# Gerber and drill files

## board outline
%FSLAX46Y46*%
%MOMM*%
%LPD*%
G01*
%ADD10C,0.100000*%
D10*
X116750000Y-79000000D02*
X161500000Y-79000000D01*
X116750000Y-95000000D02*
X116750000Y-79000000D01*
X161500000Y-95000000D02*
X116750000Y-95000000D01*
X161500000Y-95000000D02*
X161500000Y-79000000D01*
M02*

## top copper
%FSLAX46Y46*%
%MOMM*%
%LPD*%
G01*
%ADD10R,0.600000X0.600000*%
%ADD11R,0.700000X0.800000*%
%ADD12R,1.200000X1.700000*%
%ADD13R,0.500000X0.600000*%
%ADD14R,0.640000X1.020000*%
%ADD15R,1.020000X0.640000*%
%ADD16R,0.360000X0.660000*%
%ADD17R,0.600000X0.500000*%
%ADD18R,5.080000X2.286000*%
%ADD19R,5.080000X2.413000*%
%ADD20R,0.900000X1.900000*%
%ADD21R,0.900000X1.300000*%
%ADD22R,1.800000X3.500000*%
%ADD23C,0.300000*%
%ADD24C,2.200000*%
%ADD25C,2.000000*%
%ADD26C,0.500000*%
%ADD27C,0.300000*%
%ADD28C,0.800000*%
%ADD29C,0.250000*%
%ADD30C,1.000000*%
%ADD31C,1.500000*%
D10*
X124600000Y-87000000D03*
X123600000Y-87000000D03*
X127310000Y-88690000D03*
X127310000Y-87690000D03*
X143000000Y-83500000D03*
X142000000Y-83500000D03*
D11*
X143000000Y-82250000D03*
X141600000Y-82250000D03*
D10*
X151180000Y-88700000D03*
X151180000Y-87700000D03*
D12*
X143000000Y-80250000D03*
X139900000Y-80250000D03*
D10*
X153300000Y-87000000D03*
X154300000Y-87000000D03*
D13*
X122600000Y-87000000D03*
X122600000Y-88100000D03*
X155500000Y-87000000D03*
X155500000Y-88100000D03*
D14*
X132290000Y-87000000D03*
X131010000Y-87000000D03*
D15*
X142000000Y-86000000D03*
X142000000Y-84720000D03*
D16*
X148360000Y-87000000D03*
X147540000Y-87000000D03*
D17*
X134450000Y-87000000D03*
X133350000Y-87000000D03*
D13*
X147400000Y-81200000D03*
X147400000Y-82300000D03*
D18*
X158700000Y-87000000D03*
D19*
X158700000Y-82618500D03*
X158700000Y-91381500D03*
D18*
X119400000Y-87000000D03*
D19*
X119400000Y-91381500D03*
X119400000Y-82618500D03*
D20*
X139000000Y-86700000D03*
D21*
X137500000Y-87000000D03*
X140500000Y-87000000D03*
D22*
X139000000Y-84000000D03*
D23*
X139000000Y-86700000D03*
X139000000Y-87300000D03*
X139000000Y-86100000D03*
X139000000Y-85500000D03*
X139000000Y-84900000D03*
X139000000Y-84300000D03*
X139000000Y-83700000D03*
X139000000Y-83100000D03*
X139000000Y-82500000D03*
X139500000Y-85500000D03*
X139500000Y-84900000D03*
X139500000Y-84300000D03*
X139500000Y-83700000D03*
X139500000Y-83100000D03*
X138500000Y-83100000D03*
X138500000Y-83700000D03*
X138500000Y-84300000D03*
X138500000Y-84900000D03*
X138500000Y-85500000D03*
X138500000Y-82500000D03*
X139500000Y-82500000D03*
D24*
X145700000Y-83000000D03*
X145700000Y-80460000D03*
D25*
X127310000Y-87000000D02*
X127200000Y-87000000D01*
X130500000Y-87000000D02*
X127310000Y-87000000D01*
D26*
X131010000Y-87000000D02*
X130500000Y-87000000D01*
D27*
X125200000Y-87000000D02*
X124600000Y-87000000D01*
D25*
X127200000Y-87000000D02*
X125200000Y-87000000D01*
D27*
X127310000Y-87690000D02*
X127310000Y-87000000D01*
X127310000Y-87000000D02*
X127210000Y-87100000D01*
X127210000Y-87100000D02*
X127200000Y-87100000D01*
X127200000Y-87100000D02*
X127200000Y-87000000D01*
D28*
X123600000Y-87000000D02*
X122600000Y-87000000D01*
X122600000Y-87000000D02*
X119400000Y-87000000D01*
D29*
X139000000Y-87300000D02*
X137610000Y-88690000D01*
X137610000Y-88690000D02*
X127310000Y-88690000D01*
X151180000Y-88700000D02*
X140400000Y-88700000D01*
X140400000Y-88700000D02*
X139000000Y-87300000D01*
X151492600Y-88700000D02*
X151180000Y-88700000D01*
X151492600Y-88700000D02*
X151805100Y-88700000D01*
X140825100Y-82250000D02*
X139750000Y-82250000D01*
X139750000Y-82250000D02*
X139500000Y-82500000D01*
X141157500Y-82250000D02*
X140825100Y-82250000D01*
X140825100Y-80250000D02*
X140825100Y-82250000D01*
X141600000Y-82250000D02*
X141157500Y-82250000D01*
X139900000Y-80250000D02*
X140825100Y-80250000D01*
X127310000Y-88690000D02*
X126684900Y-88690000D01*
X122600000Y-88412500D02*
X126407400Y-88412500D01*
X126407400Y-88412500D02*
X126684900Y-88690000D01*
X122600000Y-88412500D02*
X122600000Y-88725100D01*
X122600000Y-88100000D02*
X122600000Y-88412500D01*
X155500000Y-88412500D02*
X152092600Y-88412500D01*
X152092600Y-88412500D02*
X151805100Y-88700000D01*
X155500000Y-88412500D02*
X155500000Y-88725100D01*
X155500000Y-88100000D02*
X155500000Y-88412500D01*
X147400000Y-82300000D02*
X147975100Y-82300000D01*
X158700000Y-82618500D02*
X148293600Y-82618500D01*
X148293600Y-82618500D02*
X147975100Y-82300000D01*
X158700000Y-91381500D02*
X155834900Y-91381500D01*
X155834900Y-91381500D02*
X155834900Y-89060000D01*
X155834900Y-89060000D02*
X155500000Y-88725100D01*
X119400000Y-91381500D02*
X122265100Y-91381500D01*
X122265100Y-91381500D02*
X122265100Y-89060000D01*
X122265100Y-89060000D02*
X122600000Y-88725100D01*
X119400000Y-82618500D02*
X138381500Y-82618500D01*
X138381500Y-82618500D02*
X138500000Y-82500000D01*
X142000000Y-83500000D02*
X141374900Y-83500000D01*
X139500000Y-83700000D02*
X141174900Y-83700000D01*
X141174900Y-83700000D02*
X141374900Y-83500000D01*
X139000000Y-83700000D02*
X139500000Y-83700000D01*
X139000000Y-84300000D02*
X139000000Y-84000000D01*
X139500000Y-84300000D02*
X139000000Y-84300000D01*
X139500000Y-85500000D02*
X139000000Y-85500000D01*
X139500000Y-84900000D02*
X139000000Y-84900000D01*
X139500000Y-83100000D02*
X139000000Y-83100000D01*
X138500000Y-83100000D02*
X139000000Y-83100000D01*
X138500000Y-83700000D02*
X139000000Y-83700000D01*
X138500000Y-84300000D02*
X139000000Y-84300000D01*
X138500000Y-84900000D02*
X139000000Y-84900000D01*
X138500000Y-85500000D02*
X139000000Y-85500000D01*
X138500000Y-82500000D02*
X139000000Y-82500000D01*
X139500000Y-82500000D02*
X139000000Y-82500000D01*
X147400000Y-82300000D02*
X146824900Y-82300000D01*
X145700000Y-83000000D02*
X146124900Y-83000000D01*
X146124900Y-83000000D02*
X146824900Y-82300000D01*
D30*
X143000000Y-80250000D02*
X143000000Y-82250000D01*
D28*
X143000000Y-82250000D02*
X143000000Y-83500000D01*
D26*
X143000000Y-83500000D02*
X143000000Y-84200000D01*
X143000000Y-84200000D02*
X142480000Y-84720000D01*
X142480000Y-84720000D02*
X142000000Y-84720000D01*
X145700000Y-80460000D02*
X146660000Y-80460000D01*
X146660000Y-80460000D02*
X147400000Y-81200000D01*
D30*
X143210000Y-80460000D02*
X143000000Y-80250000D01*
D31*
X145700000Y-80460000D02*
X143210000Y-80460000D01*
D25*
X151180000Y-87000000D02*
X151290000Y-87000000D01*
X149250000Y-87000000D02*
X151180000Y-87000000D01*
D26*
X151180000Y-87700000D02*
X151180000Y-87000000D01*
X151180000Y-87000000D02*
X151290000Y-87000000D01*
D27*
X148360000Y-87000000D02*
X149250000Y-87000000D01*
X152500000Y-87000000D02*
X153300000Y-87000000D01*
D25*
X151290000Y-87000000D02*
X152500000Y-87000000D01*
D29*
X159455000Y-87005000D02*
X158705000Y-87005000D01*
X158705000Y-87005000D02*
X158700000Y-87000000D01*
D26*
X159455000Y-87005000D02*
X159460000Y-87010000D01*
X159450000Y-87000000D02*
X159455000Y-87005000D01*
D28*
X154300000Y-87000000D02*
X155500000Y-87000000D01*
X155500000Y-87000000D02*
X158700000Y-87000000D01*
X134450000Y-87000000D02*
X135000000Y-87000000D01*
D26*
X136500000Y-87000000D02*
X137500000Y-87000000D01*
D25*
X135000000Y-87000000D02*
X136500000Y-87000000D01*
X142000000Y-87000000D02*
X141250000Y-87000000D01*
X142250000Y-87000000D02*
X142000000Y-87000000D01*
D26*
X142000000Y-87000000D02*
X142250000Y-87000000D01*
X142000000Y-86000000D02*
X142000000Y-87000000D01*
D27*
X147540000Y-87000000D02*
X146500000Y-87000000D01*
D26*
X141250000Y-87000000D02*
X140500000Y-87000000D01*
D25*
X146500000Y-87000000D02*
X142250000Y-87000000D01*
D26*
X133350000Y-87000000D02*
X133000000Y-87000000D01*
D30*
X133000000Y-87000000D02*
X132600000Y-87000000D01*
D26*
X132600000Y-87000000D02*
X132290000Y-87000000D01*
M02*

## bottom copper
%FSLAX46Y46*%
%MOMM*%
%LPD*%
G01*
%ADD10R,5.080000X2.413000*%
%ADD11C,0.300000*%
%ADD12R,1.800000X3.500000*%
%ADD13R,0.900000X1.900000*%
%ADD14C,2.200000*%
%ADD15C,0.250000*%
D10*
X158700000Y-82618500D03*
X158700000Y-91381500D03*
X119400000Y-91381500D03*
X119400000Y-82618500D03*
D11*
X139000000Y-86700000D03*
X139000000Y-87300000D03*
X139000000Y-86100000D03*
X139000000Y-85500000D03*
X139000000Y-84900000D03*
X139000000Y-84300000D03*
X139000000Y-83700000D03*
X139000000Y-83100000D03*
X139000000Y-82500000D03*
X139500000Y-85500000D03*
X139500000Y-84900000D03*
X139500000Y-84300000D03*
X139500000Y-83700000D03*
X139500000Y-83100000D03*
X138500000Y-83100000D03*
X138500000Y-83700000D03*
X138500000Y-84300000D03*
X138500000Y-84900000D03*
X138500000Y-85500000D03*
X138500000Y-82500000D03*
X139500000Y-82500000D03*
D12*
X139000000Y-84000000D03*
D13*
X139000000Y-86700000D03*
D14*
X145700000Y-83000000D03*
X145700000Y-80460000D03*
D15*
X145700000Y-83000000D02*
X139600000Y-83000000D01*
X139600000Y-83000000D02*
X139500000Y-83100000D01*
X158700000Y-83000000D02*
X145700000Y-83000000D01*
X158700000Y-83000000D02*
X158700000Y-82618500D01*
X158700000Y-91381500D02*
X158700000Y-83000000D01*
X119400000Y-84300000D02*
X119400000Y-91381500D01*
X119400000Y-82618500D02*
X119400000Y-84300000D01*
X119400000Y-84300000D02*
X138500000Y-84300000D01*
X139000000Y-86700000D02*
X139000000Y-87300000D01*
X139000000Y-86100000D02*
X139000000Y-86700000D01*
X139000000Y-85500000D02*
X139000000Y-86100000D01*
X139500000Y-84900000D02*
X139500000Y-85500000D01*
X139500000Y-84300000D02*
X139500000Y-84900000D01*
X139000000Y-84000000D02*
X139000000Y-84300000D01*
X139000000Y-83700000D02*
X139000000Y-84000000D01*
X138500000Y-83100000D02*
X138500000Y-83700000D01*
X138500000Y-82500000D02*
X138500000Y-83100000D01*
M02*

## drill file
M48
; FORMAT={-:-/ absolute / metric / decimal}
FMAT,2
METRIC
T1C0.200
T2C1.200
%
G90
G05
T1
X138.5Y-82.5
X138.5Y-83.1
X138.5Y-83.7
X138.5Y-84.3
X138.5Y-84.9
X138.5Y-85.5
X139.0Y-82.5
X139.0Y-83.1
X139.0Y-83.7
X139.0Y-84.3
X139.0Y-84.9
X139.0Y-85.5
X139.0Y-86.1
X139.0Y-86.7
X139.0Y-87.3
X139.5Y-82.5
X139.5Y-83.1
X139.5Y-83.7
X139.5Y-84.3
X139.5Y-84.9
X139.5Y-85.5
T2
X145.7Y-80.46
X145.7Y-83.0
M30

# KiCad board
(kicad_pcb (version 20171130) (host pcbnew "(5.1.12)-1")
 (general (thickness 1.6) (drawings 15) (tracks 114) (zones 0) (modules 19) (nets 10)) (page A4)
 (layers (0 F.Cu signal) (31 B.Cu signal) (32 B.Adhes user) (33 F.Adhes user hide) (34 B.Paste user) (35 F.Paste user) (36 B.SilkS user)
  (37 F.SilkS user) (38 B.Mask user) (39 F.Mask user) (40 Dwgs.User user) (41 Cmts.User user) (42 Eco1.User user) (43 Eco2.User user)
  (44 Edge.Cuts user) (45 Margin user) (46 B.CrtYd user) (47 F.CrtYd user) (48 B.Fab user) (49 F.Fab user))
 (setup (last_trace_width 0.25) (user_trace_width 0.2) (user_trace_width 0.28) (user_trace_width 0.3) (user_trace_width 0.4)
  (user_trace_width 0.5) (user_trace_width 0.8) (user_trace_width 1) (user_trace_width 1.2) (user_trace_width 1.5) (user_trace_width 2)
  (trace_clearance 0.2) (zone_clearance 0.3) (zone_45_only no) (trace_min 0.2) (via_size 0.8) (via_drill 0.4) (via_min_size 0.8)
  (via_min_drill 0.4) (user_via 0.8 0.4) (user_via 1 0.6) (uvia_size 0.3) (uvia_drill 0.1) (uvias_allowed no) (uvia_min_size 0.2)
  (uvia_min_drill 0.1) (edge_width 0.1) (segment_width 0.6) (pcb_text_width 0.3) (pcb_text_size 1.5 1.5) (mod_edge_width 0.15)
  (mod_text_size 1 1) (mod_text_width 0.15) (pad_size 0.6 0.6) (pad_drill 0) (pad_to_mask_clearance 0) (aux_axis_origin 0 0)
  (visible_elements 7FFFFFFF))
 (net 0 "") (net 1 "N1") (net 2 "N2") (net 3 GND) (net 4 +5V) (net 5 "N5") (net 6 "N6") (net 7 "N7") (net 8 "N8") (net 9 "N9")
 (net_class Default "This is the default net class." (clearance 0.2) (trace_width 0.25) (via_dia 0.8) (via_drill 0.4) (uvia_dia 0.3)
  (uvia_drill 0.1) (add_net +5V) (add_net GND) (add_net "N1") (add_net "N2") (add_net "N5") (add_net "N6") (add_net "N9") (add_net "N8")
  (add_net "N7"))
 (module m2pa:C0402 (layer F.Cu) (at 124.6 87 180)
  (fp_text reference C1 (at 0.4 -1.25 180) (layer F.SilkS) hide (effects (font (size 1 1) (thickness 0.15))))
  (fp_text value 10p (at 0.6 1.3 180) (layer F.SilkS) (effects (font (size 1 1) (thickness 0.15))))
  (pad 1 smd rect (at 0 0 180) (size 0.6 0.6) (layers F.Cu F.Paste F.Mask) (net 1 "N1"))
  (pad 2 smd rect (at 1 0 180) (size 0.6 0.6) (layers F.Cu F.Paste F.Mask) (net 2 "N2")))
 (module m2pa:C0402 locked (layer F.Cu) (at 127.31 88.69 90)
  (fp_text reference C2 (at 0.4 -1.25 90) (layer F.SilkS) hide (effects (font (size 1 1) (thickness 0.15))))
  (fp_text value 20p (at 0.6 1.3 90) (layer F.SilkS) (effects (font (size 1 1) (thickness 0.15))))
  (pad 1 smd rect (at 0 0 90) (size 0.6 0.6) (layers F.Cu F.Paste F.Mask) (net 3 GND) (zone_connect 2))
  (pad 2 smd rect (at 1 0 90) (size 0.6 0.6) (layers F.Cu F.Paste F.Mask) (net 1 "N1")))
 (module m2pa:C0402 (layer F.Cu) (at 143 83.5 180)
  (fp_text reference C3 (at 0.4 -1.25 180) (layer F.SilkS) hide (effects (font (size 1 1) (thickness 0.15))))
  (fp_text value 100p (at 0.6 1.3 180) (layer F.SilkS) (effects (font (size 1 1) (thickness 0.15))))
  (pad 1 smd rect (at 0 0 180) (size 0.6 0.6) (layers F.Cu F.Paste F.Mask) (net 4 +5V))
  (pad 2 smd rect (at 1 0 180) (size 0.6 0.6) (layers F.Cu F.Paste F.Mask) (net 3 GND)))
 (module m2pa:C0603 (layer F.Cu) (at 143 82.25 180)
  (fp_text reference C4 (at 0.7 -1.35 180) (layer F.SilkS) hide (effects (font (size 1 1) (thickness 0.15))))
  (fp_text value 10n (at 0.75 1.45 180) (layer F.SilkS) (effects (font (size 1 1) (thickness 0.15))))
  (pad 1 smd rect (at 0 0 180) (size 0.7 0.8) (layers F.Cu F.Paste F.Mask) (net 4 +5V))
  (pad 2 smd rect (at 1.4 0 180) (size 0.7 0.8) (layers F.Cu F.Paste F.Mask) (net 3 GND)))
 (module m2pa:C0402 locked (layer F.Cu) (at 151.18 88.7 90)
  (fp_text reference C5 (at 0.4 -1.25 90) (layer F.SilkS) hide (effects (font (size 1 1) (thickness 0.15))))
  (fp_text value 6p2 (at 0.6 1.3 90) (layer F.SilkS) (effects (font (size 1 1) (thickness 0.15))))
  (pad 1 smd rect (at 0 0 90) (size 0.6 0.6) (layers F.Cu F.Paste F.Mask) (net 3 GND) (zone_connect 2))
  (pad 2 smd rect (at 1 0 90) (size 0.6 0.6) (layers F.Cu F.Paste F.Mask) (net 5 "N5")))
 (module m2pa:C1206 (layer F.Cu) (at 143 80.25 180)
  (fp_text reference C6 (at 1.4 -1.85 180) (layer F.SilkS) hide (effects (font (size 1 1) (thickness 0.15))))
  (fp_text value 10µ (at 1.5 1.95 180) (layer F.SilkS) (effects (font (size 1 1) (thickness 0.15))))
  (pad 1 smd rect (at 0 0 180) (size 1.2 1.7) (layers F.Cu F.Paste F.Mask) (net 4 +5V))
  (pad 2 smd rect (at 3.1 0 180) (size 1.2 1.7) (layers F.Cu F.Paste F.Mask) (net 3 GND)))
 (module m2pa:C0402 (layer F.Cu) (at 153.3 87)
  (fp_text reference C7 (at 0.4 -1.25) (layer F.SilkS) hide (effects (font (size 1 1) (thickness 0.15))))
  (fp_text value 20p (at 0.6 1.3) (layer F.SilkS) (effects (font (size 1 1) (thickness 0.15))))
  (pad 1 smd rect (at 0 0) (size 0.6 0.6) (layers F.Cu F.Paste F.Mask) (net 5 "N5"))
  (pad 2 smd rect (at 1 0) (size 0.6 0.6) (layers F.Cu F.Paste F.Mask) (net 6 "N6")))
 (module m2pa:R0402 (layer F.Cu) (at 122.6 87 270)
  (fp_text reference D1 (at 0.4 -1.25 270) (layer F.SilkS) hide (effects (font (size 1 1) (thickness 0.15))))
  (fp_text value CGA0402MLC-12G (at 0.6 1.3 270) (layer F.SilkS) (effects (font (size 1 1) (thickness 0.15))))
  (pad 1 smd rect (at 0 0 270) (size 0.6 0.5) (layers F.Cu F.Paste F.Mask) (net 2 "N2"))
  (pad 2 smd rect (at 1.1 0 270) (size 0.6 0.5) (layers F.Cu F.Paste F.Mask) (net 3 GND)))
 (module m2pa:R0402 (layer F.Cu) (at 155.5 87 270)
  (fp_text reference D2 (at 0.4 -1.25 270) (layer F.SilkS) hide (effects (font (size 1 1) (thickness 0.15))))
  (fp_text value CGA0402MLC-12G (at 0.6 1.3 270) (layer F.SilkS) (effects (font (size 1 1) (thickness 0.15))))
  (pad 1 smd rect (at 0 0 270) (size 0.6 0.5) (layers F.Cu F.Paste F.Mask) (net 6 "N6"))
  (pad 2 smd rect (at 1.1 0 270) (size 0.6 0.5) (layers F.Cu F.Paste F.Mask) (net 3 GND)))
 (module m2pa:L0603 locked (layer F.Cu) (at 132.29 87 180)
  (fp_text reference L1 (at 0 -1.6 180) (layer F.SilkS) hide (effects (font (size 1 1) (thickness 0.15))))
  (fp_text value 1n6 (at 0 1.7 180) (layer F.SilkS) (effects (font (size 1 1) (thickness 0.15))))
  (pad 1 smd rect (at 0 0 180) (size 0.64 1.02) (layers F.Cu F.Paste F.Mask) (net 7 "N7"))
  (pad 2 smd rect (at 1.28 0 180) (size 0.64 1.02) (layers F.Cu F.Paste F.Mask) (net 1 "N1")))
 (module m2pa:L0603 (layer F.Cu) (at 142 86 90)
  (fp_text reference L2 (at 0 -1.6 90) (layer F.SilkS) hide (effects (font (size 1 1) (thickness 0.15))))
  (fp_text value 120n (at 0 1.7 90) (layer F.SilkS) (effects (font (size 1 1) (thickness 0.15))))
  (pad 1 smd rect (at 0 0 90) (size 0.64 1.02) (layers F.Cu F.Paste F.Mask) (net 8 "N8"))
  (pad 2 smd rect (at 1.28 0 90) (size 0.64 1.02) (layers F.Cu F.Paste F.Mask) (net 4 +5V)))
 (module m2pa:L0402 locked (layer F.Cu) (at 148.36 87 180)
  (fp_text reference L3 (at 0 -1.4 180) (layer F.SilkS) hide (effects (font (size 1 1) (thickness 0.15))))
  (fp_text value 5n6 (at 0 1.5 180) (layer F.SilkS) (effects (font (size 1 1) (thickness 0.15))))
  (pad 1 smd rect (at 0 0 180) (size 0.36 0.66) (layers F.Cu F.Paste F.Mask) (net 5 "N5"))
  (pad 2 smd rect (at 0.82 0 180) (size 0.36 0.66) (layers F.Cu F.Paste F.Mask) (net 8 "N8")))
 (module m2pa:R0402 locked (layer F.Cu) (at 134.45 87 180)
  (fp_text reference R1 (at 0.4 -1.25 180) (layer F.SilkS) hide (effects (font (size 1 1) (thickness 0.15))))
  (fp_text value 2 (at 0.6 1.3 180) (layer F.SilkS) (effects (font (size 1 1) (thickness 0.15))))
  (pad 1 smd rect (at 0 0 180) (size 0.6 0.5) (layers F.Cu F.Paste F.Mask) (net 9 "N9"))
  (pad 2 smd rect (at 1.1 0 180) (size 0.6 0.5) (layers F.Cu F.Paste F.Mask) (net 7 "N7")))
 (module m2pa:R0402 (layer F.Cu) (at 147.4 81.2 270)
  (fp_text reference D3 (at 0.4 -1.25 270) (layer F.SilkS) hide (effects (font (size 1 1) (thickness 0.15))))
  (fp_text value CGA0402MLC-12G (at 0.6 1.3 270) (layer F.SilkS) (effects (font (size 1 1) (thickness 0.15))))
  (pad 1 smd rect (at 0 0 270) (size 0.6 0.5) (layers F.Cu F.Paste F.Mask) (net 4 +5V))
  (pad 2 smd rect (at 1.1 0 270) (size 0.6 0.5) (layers F.Cu F.Paste F.Mask) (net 3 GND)))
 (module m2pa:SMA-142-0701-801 (layer F.Cu) (at 158.7 87 270)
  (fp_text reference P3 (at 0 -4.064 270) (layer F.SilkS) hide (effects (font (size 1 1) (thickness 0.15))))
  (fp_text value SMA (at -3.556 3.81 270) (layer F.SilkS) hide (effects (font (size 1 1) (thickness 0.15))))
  (pad 1 smd rect (at 0 0 270) (size 2.286 5.08) (layers F.Cu F.Mask) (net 6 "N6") (zone_connect 2))
  (pad 2 smd rect (at -4.3815 0 270) (size 2.413 5.08) (layers F.Cu F.Mask) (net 3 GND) (zone_connect 2))
  (pad 3 smd rect (at 4.3815 0 270) (size 2.413 5.08) (layers F.Cu F.Mask) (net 3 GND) (zone_connect 2))
  (pad 4 smd rect (at -4.3815 0 270) (size 2.413 5.08) (layers B.Cu B.Mask) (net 3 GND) (zone_connect 2))
  (pad 5 smd rect (at 4.3815 0 270) (size 2.413 5.08) (layers B.Cu B.Mask) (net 3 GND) (zone_connect 2)))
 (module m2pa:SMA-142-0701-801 (layer F.Cu) (at 119.4 87 90)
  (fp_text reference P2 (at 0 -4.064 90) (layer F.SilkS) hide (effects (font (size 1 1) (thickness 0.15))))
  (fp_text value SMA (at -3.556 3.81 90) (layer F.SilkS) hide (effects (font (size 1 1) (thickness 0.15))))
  (pad 1 smd rect (at 0 0 90) (size 2.286 5.08) (layers F.Cu F.Mask) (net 2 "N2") (zone_connect 2))
  (pad 2 smd rect (at -4.3815 0 90) (size 2.413 5.08) (layers F.Cu F.Mask) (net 3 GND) (zone_connect 2))
  (pad 3 smd rect (at 4.3815 0 90) (size 2.413 5.08) (layers F.Cu F.Mask) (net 3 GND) (zone_connect 2))
  (pad 4 smd rect (at -4.3815 0 90) (size 2.413 5.08) (layers B.Cu B.Mask) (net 3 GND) (zone_connect 2))
  (pad 5 smd rect (at 4.3815 0 90) (size 2.413 5.08) (layers B.Cu B.Mask) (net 3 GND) (zone_connect 2)))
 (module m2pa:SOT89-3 (layer F.Cu) (at 139 87)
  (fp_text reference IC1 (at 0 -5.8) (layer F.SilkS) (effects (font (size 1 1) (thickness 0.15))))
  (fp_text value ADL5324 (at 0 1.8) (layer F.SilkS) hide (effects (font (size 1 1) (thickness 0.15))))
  (pad 2 smd rect (at 0 -0.3 180) (size 0.9 1.9) (layers F.Cu F.Paste F.Mask) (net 3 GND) (zone_connect 2))
  (pad 1 smd rect (at -1.5 0 180) (size 0.9 1.3) (layers F.Cu F.Paste F.Mask) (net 9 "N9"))
  (pad 3 smd rect (at 1.5 0 180) (size 0.9 1.3) (layers F.Cu F.Paste F.Mask) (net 8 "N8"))
  (pad 2 smd rect (at 0 -3 180) (size 1.8 3.5) (layers F.Cu F.Paste F.Mask) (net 3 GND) (zone_connect 2))
  (pad 2 thru_hole circle (at 0 -0.3 180) (size 0.3 0.3) (drill 0.2) (layers *.Cu F.SilkS F.Mask) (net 3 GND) (zone_connect 2))
  (pad 2 thru_hole circle (at 0 0.3 180) (size 0.3 0.3) (drill 0.2) (layers *.Cu F.SilkS F.Mask) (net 3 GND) (zone_connect 2))
  (pad 2 thru_hole circle (at 0 -0.9 180) (size 0.3 0.3) (drill 0.2) (layers *.Cu F.SilkS F.Mask) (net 3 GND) (zone_connect 2))
  (pad 2 thru_hole circle (at 0 -1.5 180) (size 0.3 0.3) (drill 0.2) (layers *.Cu F.SilkS F.Mask) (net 3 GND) (zone_connect 2))
  (pad 2 thru_hole circle (at 0 -2.1 180) (size 0.3 0.3) (drill 0.2) (layers *.Cu F.SilkS F.Mask) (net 3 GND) (zone_connect 2))
  (pad 2 thru_hole circle (at 0 -2.7 180) (size 0.3 0.3) (drill 0.2) (layers *.Cu F.SilkS F.Mask) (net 3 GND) (zone_connect 2))
  (pad 2 thru_hole circle (at 0 -3.3 180) (size 0.3 0.3) (drill 0.2) (layers *.Cu F.SilkS F.Mask) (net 3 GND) (zone_connect 2))
  (pad 2 thru_hole circle (at 0 -3.9 180) (size 0.3 0.3) (drill 0.2) (layers *.Cu F.SilkS F.Mask) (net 3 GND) (zone_connect 2))
  (pad 2 thru_hole circle (at 0 -4.5 180) (size 0.3 0.3) (drill 0.2) (layers *.Cu F.SilkS F.Mask) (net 3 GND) (zone_connect 2))
  (pad 2 thru_hole circle (at 0.5 -1.5 180) (size 0.3 0.3) (drill 0.2) (layers *.Cu F.SilkS F.Mask) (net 3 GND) (zone_connect 2))
  (pad 2 thru_hole circle (at 0.5 -2.1 180) (size 0.3 0.3) (drill 0.2) (layers *.Cu F.SilkS F.Mask) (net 3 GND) (zone_connect 2))
  (pad 2 thru_hole circle (at 0.5 -2.7 180) (size 0.3 0.3) (drill 0.2) (layers *.Cu F.SilkS F.Mask) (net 3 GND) (zone_connect 2))
  (pad 2 thru_hole circle (at 0.5 -3.3 180) (size 0.3 0.3) (drill 0.2) (layers *.Cu F.SilkS F.Mask) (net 3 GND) (zone_connect 2))
  (pad 2 thru_hole circle (at 0.5 -3.9 180) (size 0.3 0.3) (drill 0.2) (layers *.Cu F.SilkS F.Mask) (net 3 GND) (zone_connect 2))
  (pad 2 thru_hole circle (at -0.5 -3.9 180) (size 0.3 0.3) (drill 0.2) (layers *.Cu F.SilkS F.Mask) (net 3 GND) (zone_connect 2))
  (pad 2 thru_hole circle (at -0.5 -3.3 180) (size 0.3 0.3) (drill 0.2) (layers *.Cu F.SilkS F.Mask) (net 3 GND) (zone_connect 2))
  (pad 2 thru_hole circle (at -0.5 -2.7 180) (size 0.3 0.3) (drill 0.2) (layers *.Cu F.SilkS F.Mask) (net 3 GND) (zone_connect 2))
  (pad 2 thru_hole circle (at -0.5 -2.1 180) (size 0.3 0.3) (drill 0.2) (layers *.Cu F.SilkS F.Mask) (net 3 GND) (zone_connect 2))
  (pad 2 thru_hole circle (at -0.5 -1.5 180) (size 0.3 0.3) (drill 0.2) (layers *.Cu F.SilkS F.Mask) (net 3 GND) (zone_connect 2))
  (pad 2 thru_hole circle (at -0.5 -4.5 180) (size 0.3 0.3) (drill 0.2) (layers *.Cu F.SilkS F.Mask) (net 3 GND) (zone_connect 2))
  (pad 2 thru_hole circle (at 0.5 -4.5 180) (size 0.3 0.3) (drill 0.2) (layers *.Cu F.SilkS F.Mask) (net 3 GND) (zone_connect 2))
  (pad 2 smd rect (at 0 -3 180) (size 1.8 3.5) (layers B.Cu) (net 3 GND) (zone_connect 2))
  (pad 2 smd rect (at 0 -0.3 180) (size 0.9 1.9) (layers B.Cu) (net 3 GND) (zone_connect 2)))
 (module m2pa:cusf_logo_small (layer F.Cu) (at 130 90.5 270)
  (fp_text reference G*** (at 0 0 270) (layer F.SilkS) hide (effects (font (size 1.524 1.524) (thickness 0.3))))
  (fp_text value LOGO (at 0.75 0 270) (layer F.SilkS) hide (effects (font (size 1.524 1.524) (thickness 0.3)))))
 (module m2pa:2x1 (layer F.Cu) (at 145.7 83 90)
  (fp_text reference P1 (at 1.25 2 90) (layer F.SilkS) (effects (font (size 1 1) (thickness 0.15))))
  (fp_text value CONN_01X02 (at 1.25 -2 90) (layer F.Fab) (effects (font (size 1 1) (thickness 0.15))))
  (pad 1 thru_hole circle (at 0 0 90) (size 2.2 2.2) (drill 1.2) (layers *.Cu *.Mask F.SilkS) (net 3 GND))
  (pad 2 thru_hole circle (at 2.54 0 90) (size 2.2 2.2) (drill 1.2) (layers *.Cu *.Mask F.SilkS) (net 4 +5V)))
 (gr_line (start 116.75 79) (end 161.5 79) (angle 90) (layer Edge.Cuts) (width 0.1))
 (gr_line (start 116.75 95) (end 116.75 79) (angle 90) (layer Edge.Cuts) (width 0.1))
 (gr_line (start 161.5 95) (end 116.75 95) (angle 90) (layer Edge.Cuts) (width 0.1))
 (gr_line (start 161.5 95) (end 161.5 79) (angle 90) (layer Edge.Cuts) (width 0.1))
 (segment (start 127.31 87) (end 127.2 87) (width 2) (layer F.Cu) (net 1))
 (segment (start 130.5 87) (end 127.31 87) (width 2) (layer F.Cu) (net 1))
 (segment (start 131.01 87) (end 130.5 87) (width 0.5) (layer F.Cu) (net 1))
 (segment (start 125.2 87) (end 124.6 87) (width 0.3) (layer F.Cu) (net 1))
 (segment (start 127.2 87) (end 125.2 87) (width 2) (layer F.Cu) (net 1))
 (segment (start 127.31 87.69) (end 127.31 87) (width 0.3) (layer F.Cu) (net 1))
 (segment (start 127.31 87) (end 127.21 87.1) (width 0.3) (layer F.Cu) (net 1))
 (segment (start 127.21 87.1) (end 127.2 87.1) (width 0.3) (layer F.Cu) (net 1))
 (segment (start 127.2 87.1) (end 127.2 87) (width 0.3) (layer F.Cu) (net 1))
 (segment (start 123.6 87) (end 122.6 87) (width 0.8) (layer F.Cu) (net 2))
 (segment (start 122.6 87) (end 119.4 87) (width 0.8) (layer F.Cu) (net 2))
 (segment (start 139 87.3) (end 137.61 88.69) (width 0.25) (layer F.Cu) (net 3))
 (segment (start 137.61 88.69) (end 127.31 88.69) (width 0.25) (layer F.Cu) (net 3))
 (segment (start 151.18 88.7) (end 140.4 88.7) (width 0.25) (layer F.Cu) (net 3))
 (segment (start 140.4 88.7) (end 139 87.3) (width 0.25) (layer F.Cu) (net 3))
 (segment (start 151.4926 88.7) (end 151.18 88.7) (width 0.25) (layer F.Cu) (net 3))
 (segment (start 151.4926 88.7) (end 151.8051 88.7) (width 0.25) (layer F.Cu) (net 3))
 (segment (start 140.8251 82.25) (end 139.75 82.25) (width 0.25) (layer F.Cu) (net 3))
 (segment (start 139.75 82.25) (end 139.5 82.5) (width 0.25) (layer F.Cu) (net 3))
 (segment (start 141.1575 82.25) (end 140.8251 82.25) (width 0.25) (layer F.Cu) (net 3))
 (segment (start 140.8251 80.25) (end 140.8251 82.25) (width 0.25) (layer F.Cu) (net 3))
 (segment (start 141.6 82.25) (end 141.1575 82.25) (width 0.25) (layer F.Cu) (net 3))
 (segment (start 139.9 80.25) (end 140.8251 80.25) (width 0.25) (layer F.Cu) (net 3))
 (segment (start 127.31 88.69) (end 126.6849 88.69) (width 0.25) (layer F.Cu) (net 3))
 (segment (start 122.6 88.4125) (end 126.4074 88.4125) (width 0.25) (layer F.Cu) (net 3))
 (segment (start 126.4074 88.4125) (end 126.6849 88.69) (width 0.25) (layer F.Cu) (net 3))
 (segment (start 122.6 88.4125) (end 122.6 88.7251) (width 0.25) (layer F.Cu) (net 3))
 (segment (start 122.6 88.1) (end 122.6 88.4125) (width 0.25) (layer F.Cu) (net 3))
 (segment (start 155.5 88.4125) (end 152.0926 88.4125) (width 0.25) (layer F.Cu) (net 3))
 (segment (start 152.0926 88.4125) (end 151.8051 88.7) (width 0.25) (layer F.Cu) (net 3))
 (segment (start 155.5 88.4125) (end 155.5 88.7251) (width 0.25) (layer F.Cu) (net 3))
 (segment (start 155.5 88.1) (end 155.5 88.4125) (width 0.25) (layer F.Cu) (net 3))
 (segment (start 145.7 83) (end 139.6 83) (width 0.25) (layer B.Cu) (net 3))
 (segment (start 139.6 83) (end 139.5 83.1) (width 0.25) (layer B.Cu) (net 3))
 (segment (start 158.7 83) (end 145.7 83) (width 0.25) (layer B.Cu) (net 3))
 (segment (start 147.4 82.3) (end 147.9751 82.3) (width 0.25) (layer F.Cu) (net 3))
 (segment (start 158.7 82.6185) (end 148.2936 82.6185) (width 0.25) (layer F.Cu) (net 3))
 (segment (start 148.2936 82.6185) (end 147.9751 82.3) (width 0.25) (layer F.Cu) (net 3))
 (segment (start 158.7 91.3815) (end 155.8349 91.3815) (width 0.25) (layer F.Cu) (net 3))
 (segment (start 155.8349 91.3815) (end 155.8349 89.06) (width 0.25) (layer F.Cu) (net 3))
 (segment (start 155.8349 89.06) (end 155.5 88.7251) (width 0.25) (layer F.Cu) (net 3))
 (segment (start 158.7 83) (end 158.7 82.6185) (width 0.25) (layer B.Cu) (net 3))
 (segment (start 158.7 91.3815) (end 158.7 83) (width 0.25) (layer B.Cu) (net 3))
 (segment (start 119.4 91.3815) (end 122.2651 91.3815) (width 0.25) (layer F.Cu) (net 3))
 (segment (start 122.2651 91.3815) (end 122.2651 89.06) (width 0.25) (layer F.Cu) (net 3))
 (segment (start 122.2651 89.06) (end 122.6 88.7251) (width 0.25) (layer F.Cu) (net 3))
 (segment (start 119.4 82.6185) (end 138.3815 82.6185) (width 0.25) (layer F.Cu) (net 3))
 (segment (start 138.3815 82.6185) (end 138.5 82.5) (width 0.25) (layer F.Cu) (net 3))
 (segment (start 119.4 84.3) (end 119.4 91.3815) (width 0.25) (layer B.Cu) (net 3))
 (segment (start 119.4 82.6185) (end 119.4 84.3) (width 0.25) (layer B.Cu) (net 3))
 (segment (start 119.4 84.3) (end 138.5 84.3) (width 0.25) (layer B.Cu) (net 3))
 (segment (start 142 83.5) (end 141.3749 83.5) (width 0.25) (layer F.Cu) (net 3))
 (segment (start 139.5 83.7) (end 141.1749 83.7) (width 0.25) (layer F.Cu) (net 3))
 (segment (start 141.1749 83.7) (end 141.3749 83.5) (width 0.25) (layer F.Cu) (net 3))
 (segment (start 139 83.7) (end 139.5 83.7) (width 0.25) (layer F.Cu) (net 3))
 (segment (start 139 84.3) (end 139 84) (width 0.25) (layer F.Cu) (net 3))
 (segment (start 139.5 84.3) (end 139 84.3) (width 0.25) (layer F.Cu) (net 3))
 (segment (start 139 86.7) (end 139 87.3) (width 0.25) (layer B.Cu) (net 3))
 (segment (start 139 86.1) (end 139 86.7) (width 0.25) (layer B.Cu) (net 3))
 (segment (start 139 85.5) (end 139 86.1) (width 0.25) (layer B.Cu) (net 3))
 (segment (start 139.5 84.9) (end 139.5 85.5) (width 0.25) (layer B.Cu) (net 3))
 (segment (start 139.5 84.3) (end 139.5 84.9) (width 0.25) (layer B.Cu) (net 3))
 (segment (start 139 84) (end 139 84.3) (width 0.25) (layer B.Cu) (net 3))
 (segment (start 139 83.7) (end 139 84) (width 0.25) (layer B.Cu) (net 3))
 (segment (start 138.5 83.1) (end 138.5 83.7) (width 0.25) (layer B.Cu) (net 3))
 (segment (start 138.5 82.5) (end 138.5 83.1) (width 0.25) (layer B.Cu) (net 3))
 (segment (start 139.5 85.5) (end 139 85.5) (width 0.25) (layer F.Cu) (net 3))
 (segment (start 139.5 84.9) (end 139 84.9) (width 0.25) (layer F.Cu) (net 3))
 (segment (start 139.5 83.1) (end 139 83.1) (width 0.25) (layer F.Cu) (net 3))
 (segment (start 138.5 83.1) (end 139 83.1) (width 0.25) (layer F.Cu) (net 3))
 (segment (start 138.5 83.7) (end 139 83.7) (width 0.25) (layer F.Cu) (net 3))
 (segment (start 138.5 84.3) (end 139 84.3) (width 0.25) (layer F.Cu) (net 3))
 (segment (start 138.5 84.9) (end 139 84.9) (width 0.25) (layer F.Cu) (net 3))
 (segment (start 138.5 85.5) (end 139 85.5) (width 0.25) (layer F.Cu) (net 3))
 (segment (start 138.5 82.5) (end 139 82.5) (width 0.25) (layer F.Cu) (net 3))
 (segment (start 139.5 82.5) (end 139 82.5) (width 0.25) (layer F.Cu) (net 3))
 (segment (start 147.4 82.3) (end 146.8249 82.3) (width 0.25) (layer F.Cu) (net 3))
 (segment (start 145.7 83) (end 146.1249 83) (width 0.25) (layer F.Cu) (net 3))
 (segment (start 146.1249 83) (end 146.8249 82.3) (width 0.25) (layer F.Cu) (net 3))
 (segment (start 143 80.25) (end 143 82.25) (width 1) (layer F.Cu) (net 4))
 (segment (start 143 82.25) (end 143 83.5) (width 0.8) (layer F.Cu) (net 4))
 (segment (start 143 83.5) (end 143 84.2) (width 0.5) (layer F.Cu) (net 4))
 (segment (start 143 84.2) (end 142.48 84.72) (width 0.5) (layer F.Cu) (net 4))
 (segment (start 142.48 84.72) (end 142 84.72) (width 0.5) (layer F.Cu) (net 4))
 (segment (start 145.7 80.46) (end 146.66 80.46) (width 0.5) (layer F.Cu) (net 4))
 (segment (start 146.66 80.46) (end 147.4 81.2) (width 0.5) (layer F.Cu) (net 4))
 (segment (start 143.21 80.46) (end 143 80.25) (width 1) (layer F.Cu) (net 4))
 (segment (start 145.7 80.46) (end 143.21 80.46) (width 1.5) (layer F.Cu) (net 4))
 (segment (start 151.18 87) (end 151.29 87) (width 2) (layer F.Cu) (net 5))
 (segment (start 149.25 87) (end 151.18 87) (width 2) (layer F.Cu) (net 5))
 (segment (start 151.18 87.7) (end 151.18 87) (width 0.5) (layer F.Cu) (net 5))
 (segment (start 151.18 87) (end 151.29 87) (width 0.5) (layer F.Cu) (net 5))
 (segment (start 148.36 87) (end 149.25 87) (width 0.3) (layer F.Cu) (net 5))
 (segment (start 152.5 87) (end 153.3 87) (width 0.3) (layer F.Cu) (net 5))
 (segment (start 151.29 87) (end 152.5 87) (width 2) (layer F.Cu) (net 5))
 (segment (start 159.455 87.005) (end 158.705 87.005) (width 0.25) (layer F.Cu) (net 6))
 (segment (start 158.705 87.005) (end 158.7 87) (width 0.25) (layer F.Cu) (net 6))
 (segment (start 159.455 87.005) (end 159.46 87.01) (width 0.5) (layer F.Cu) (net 6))
 (segment (start 159.45 87) (end 159.455 87.005) (width 0.5) (layer F.Cu) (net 6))
 (segment (start 154.3 87) (end 155.5 87) (width 0.8) (layer F.Cu) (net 6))
 (segment (start 155.5 87) (end 158.7 87) (width 0.8) (layer F.Cu) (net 6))
 (segment (start 134.45 87) (end 135 87) (width 0.8) (layer F.Cu) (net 9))
 (segment (start 136.5 87) (end 137.5 87) (width 0.5) (layer F.Cu) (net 9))
 (segment (start 135 87) (end 136.5 87) (width 2) (layer F.Cu) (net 9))
 (segment (start 142 87) (end 141.25 87) (width 2) (layer F.Cu) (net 8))
 (segment (start 142.25 87) (end 142 87) (width 2) (layer F.Cu) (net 8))
 (segment (start 142 87) (end 142.25 87) (width 0.5) (layer F.Cu) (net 8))
 (segment (start 142 86) (end 142 87) (width 0.5) (layer F.Cu) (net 8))
 (segment (start 147.54 87) (end 146.5 87) (width 0.3) (layer F.Cu) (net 8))
 (segment (start 141.25 87) (end 140.5 87) (width 0.5) (layer F.Cu) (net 8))
 (segment (start 146.5 87) (end 142.25 87) (width 2) (layer F.Cu) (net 8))
 (segment (start 133.35 87) (end 133 87) (width 0.5) (layer F.Cu) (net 7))
 (segment (start 133 87) (end 132.6 87) (width 1) (layer F.Cu) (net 7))
 (segment (start 132.6 87) (end 132.29 87) (width 0.5) (layer F.Cu) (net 7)))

